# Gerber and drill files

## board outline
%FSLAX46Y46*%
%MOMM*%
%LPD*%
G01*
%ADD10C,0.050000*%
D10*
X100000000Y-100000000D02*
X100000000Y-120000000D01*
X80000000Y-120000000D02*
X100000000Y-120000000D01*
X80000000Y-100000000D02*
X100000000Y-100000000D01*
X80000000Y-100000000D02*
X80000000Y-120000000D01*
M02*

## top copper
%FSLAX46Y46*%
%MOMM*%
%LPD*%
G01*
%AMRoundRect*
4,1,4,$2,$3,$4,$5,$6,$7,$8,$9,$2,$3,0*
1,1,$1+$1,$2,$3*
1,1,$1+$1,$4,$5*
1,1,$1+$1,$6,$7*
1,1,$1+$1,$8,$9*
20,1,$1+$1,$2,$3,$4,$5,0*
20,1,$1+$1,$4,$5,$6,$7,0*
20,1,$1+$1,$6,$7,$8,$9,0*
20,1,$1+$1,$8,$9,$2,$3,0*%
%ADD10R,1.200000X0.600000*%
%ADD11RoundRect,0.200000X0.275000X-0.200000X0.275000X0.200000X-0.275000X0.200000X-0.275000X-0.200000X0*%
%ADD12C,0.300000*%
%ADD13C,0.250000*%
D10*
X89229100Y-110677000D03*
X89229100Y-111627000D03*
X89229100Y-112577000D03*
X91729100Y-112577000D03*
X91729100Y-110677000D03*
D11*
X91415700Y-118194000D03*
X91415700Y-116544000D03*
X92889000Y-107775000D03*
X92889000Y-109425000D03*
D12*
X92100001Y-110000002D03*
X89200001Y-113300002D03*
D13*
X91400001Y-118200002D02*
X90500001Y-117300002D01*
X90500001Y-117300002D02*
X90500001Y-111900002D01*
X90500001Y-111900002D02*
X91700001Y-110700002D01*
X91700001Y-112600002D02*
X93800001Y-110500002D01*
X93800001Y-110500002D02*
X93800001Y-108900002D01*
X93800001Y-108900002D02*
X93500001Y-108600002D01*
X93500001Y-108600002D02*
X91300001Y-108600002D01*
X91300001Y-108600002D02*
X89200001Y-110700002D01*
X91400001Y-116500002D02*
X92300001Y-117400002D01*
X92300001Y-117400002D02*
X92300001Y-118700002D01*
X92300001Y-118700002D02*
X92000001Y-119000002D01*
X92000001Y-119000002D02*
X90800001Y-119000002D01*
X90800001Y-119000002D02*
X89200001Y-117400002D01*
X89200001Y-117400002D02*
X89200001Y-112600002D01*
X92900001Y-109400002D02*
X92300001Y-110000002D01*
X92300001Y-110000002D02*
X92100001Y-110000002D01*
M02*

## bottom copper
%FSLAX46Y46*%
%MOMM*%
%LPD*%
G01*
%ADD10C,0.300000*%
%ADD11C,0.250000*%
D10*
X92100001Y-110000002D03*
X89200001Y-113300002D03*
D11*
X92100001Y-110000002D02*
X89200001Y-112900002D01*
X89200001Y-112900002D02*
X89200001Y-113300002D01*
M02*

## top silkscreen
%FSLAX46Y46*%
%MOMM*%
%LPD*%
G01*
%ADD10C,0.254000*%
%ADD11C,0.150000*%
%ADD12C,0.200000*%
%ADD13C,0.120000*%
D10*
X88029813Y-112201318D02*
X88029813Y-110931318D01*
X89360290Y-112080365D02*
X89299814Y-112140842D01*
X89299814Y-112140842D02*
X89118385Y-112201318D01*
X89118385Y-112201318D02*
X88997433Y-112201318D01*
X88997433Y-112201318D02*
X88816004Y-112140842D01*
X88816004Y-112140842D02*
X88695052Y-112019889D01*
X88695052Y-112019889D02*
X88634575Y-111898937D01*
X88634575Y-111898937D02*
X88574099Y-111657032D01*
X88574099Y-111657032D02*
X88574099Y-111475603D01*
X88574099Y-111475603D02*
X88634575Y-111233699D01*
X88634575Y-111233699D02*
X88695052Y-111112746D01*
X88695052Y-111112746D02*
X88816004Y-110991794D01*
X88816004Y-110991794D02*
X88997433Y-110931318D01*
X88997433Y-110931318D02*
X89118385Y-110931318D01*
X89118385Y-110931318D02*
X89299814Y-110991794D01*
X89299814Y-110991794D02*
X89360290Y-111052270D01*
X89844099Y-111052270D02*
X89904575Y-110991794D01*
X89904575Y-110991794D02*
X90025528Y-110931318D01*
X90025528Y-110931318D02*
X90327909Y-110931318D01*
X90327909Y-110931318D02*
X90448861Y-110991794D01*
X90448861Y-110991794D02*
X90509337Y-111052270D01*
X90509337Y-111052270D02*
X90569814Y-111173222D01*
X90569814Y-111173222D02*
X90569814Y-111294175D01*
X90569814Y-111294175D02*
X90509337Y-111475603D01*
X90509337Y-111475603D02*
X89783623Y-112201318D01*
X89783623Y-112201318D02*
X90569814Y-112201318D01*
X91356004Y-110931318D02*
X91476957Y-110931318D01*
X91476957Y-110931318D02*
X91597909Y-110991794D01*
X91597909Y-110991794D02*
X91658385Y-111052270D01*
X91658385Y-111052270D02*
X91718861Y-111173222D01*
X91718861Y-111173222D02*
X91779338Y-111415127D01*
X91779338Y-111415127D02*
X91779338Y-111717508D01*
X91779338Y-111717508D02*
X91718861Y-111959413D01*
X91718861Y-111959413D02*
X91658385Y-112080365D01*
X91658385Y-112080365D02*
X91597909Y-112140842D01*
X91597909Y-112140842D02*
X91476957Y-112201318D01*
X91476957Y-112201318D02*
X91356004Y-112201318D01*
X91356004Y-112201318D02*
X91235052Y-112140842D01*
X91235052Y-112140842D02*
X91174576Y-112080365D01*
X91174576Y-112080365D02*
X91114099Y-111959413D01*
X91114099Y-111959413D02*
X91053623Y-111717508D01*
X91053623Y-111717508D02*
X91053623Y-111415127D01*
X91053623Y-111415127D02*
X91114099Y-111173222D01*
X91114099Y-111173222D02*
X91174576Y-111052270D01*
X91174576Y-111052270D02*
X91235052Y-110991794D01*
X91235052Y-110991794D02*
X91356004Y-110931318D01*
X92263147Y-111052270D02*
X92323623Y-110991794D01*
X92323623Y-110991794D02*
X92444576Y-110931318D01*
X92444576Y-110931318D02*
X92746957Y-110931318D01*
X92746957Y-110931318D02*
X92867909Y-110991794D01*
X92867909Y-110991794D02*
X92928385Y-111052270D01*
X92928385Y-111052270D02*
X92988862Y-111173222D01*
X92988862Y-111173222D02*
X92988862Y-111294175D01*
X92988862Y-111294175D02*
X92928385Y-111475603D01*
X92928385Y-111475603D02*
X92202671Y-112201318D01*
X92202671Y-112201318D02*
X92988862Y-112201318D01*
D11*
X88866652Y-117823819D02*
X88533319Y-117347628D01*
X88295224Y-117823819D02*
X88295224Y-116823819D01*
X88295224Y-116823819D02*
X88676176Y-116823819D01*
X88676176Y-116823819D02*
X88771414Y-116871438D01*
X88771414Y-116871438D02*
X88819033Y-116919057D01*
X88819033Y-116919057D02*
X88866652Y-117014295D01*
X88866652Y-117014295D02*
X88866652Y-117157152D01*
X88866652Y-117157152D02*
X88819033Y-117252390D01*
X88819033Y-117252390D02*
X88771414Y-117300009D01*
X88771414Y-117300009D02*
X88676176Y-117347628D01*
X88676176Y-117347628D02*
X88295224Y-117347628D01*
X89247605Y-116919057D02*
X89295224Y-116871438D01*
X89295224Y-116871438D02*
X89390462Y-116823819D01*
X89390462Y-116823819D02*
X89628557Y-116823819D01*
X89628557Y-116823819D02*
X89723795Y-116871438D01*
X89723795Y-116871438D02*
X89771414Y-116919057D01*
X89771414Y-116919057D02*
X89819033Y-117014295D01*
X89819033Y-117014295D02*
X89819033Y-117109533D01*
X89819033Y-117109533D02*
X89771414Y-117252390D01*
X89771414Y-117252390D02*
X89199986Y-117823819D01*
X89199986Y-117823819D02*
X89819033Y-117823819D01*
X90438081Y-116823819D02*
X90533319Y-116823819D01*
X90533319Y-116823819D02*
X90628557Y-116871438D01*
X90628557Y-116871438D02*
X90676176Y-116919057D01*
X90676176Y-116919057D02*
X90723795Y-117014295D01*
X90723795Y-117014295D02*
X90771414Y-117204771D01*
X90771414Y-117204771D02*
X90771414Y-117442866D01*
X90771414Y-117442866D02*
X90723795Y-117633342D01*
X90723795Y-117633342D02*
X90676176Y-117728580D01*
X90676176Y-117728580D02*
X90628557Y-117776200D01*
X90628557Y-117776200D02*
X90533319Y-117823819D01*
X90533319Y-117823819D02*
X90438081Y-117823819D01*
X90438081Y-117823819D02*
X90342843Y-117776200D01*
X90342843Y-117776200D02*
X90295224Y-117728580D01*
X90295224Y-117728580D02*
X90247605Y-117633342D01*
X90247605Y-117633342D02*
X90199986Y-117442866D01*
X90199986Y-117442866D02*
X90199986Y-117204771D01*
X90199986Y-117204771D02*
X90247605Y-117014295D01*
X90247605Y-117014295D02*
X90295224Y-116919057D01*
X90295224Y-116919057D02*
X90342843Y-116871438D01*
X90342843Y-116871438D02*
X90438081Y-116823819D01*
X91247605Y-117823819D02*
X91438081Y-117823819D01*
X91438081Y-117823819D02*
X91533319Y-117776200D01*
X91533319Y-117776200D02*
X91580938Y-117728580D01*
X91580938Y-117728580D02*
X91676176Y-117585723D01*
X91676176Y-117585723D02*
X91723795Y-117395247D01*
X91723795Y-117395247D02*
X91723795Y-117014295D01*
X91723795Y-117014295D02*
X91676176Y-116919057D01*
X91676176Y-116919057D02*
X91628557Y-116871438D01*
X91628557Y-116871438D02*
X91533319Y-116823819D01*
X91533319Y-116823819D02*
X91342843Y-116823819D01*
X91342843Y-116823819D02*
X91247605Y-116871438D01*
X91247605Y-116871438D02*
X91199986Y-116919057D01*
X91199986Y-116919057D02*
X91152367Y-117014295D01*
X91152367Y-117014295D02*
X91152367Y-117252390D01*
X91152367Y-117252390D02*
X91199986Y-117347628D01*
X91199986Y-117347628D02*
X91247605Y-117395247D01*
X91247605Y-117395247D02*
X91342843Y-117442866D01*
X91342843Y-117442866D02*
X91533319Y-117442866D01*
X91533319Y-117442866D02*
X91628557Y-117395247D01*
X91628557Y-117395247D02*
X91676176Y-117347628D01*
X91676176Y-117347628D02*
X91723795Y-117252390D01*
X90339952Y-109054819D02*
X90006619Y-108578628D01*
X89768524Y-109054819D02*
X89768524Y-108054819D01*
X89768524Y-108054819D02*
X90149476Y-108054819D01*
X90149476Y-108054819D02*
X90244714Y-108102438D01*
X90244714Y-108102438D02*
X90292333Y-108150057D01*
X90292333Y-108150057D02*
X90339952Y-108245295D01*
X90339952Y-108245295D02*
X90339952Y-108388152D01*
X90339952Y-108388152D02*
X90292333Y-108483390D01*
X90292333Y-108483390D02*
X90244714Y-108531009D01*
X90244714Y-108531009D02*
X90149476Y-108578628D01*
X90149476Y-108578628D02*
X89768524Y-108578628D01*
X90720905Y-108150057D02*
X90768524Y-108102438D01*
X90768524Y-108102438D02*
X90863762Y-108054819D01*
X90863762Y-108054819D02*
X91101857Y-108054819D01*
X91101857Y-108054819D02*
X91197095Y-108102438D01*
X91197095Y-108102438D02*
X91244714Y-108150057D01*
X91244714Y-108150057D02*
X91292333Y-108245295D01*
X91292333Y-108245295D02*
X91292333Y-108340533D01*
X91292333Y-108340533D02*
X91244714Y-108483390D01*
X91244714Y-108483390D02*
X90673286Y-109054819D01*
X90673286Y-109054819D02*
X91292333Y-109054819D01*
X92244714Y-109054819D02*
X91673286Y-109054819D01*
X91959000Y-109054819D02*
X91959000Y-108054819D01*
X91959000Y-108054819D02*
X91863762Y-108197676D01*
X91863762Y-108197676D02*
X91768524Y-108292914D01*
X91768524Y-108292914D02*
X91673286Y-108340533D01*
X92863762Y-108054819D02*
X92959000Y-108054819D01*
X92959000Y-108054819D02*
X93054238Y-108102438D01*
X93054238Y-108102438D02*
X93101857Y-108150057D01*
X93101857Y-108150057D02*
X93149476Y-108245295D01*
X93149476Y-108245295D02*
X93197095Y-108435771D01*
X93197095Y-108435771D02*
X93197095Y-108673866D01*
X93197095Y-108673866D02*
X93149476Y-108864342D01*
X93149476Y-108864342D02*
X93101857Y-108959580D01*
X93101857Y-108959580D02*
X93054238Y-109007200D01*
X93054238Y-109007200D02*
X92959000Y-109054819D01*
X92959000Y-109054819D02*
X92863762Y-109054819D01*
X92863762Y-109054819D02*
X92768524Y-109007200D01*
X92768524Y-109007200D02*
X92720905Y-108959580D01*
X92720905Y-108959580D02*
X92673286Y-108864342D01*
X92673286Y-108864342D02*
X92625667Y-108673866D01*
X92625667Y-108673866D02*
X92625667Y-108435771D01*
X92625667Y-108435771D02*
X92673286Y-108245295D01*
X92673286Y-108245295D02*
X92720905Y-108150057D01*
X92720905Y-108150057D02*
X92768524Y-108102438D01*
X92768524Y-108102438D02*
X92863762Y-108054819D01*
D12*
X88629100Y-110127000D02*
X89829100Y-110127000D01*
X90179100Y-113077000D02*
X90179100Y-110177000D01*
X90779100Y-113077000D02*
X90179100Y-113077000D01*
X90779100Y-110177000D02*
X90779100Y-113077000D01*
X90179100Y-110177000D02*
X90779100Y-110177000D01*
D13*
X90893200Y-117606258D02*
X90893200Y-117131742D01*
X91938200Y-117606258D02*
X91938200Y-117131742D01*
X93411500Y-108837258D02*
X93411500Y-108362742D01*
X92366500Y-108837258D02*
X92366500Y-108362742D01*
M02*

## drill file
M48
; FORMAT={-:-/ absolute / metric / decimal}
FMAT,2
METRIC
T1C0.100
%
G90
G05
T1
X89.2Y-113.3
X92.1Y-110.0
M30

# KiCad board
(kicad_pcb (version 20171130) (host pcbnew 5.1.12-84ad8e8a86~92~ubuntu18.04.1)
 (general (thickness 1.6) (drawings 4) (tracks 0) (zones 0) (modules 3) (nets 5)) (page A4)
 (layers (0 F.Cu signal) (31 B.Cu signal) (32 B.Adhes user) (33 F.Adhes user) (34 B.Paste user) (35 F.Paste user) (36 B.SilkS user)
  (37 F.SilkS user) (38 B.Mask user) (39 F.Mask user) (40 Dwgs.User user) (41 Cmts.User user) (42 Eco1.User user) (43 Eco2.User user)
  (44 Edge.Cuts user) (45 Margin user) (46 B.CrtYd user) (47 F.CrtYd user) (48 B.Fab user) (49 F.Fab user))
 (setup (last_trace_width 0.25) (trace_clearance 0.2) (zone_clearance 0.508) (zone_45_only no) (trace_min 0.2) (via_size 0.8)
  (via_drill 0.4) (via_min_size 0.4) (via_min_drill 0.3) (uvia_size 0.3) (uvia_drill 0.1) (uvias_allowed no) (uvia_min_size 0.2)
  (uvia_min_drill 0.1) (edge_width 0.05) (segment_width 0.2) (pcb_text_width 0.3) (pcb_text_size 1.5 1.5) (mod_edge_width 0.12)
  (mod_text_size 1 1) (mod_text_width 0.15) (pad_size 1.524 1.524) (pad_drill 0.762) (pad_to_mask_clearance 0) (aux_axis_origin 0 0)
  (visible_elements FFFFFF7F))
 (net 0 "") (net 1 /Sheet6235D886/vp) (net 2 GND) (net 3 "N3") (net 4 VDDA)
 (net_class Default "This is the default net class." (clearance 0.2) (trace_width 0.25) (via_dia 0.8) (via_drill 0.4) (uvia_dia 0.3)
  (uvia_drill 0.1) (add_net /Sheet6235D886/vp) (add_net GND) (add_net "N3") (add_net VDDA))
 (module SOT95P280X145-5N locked (layer F.Cu) (at 90.479100 111.627000)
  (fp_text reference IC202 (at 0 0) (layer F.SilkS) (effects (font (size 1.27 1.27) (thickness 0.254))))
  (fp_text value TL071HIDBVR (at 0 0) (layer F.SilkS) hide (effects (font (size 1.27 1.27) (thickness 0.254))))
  (fp_line (start -1.85 -1.5) (end -0.65 -1.5) (layer F.SilkS) (width 0.2))
  (fp_line (start -0.3 1.45) (end -0.3 -1.45) (layer F.SilkS) (width 0.2))
  (fp_line (start 0.3 1.45) (end -0.3 1.45) (layer F.SilkS) (width 0.2))
  (fp_line (start 0.3 -1.45) (end 0.3 1.45) (layer F.SilkS) (width 0.2))
  (fp_line (start -0.3 -1.45) (end 0.3 -1.45) (layer F.SilkS) (width 0.2))
  (pad 1 smd rect (at -1.25 -0.95 90.000000) (size 0.6 1.2) (layers F.Cu F.Mask F.Paste) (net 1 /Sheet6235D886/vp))
  (pad 2 smd rect (at -1.25 0 90.000000) (size 0.6 1.2) (layers F.Cu F.Mask F.Paste) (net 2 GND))
  (pad 3 smd rect (at -1.25 0.95 90.000000) (size 0.6 1.2) (layers F.Cu F.Mask F.Paste) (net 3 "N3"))
  (pad 4 smd rect (at 1.25 0.95 90.000000) (size 0.6 1.2) (layers F.Cu F.Mask F.Paste) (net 1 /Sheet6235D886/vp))
  (pad 5 smd rect (at 1.25 -0.95 90.000000) (size 0.6 1.2) (layers F.Cu F.Mask F.Paste) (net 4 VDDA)))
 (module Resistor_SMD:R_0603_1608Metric (layer F.Cu) (at 91.415700 117.369000 90.000000)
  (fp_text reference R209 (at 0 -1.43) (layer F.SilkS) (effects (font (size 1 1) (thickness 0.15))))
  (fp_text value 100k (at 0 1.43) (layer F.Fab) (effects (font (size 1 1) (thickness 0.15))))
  (fp_line (start -0.237258 -0.5225) (end 0.237258 -0.5225) (layer F.SilkS) (width 0.12))
  (fp_line (start -0.237258 0.5225) (end 0.237258 0.5225) (layer F.SilkS) (width 0.12))
  (pad 1 smd roundrect (at -0.825 0 90.000000) (size 0.8 0.95) (layers F.Cu F.Mask F.Paste) (roundrect_rratio 0.25) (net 4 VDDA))
  (pad 2 smd roundrect (at 0.825 0 90.000000) (size 0.8 0.95) (layers F.Cu F.Mask F.Paste) (roundrect_rratio 0.25) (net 3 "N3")))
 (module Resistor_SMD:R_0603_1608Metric (layer F.Cu) (at 92.889000 108.600000 90.000000)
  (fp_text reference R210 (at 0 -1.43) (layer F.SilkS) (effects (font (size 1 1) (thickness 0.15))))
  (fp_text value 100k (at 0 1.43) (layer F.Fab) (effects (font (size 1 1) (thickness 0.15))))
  (fp_line (start -0.237258 0.5225) (end 0.237258 0.5225) (layer F.SilkS) (width 0.12))
  (fp_line (start -0.237258 -0.5225) (end 0.237258 -0.5225) (layer F.SilkS) (width 0.12))
  (pad 2 smd roundrect (at 0.825 0 90.000000) (size 0.8 0.95) (layers F.Cu F.Mask F.Paste) (roundrect_rratio 0.25) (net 2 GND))
  (pad 1 smd roundrect (at -0.825 0 90.000000) (size 0.8 0.95) (layers F.Cu F.Mask F.Paste) (roundrect_rratio 0.25) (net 3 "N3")))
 (gr_line (start 100 100) (end 100 120) (layer Edge.Cuts) (width 0.05))
 (gr_line (start 80 120) (end 100 120) (layer Edge.Cuts) (width 0.05))
 (gr_line (start 80 100) (end 100 100) (layer Edge.Cuts) (width 0.05))
 (gr_line (start 80 100) (end 80 120) (layer Edge.Cuts) (width 0.05))
 (segment (start 91.400001 118.200002) (end 90.500001 117.300002) (width 0.250000) (layer F.Cu) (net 4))
 (segment (start 90.500001 117.300002) (end 90.500001 111.900002) (width 0.250000) (layer F.Cu) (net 4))
 (segment (start 90.500001 111.900002) (end 91.700001 110.700002) (width 0.250000) (layer F.Cu) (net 4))
 (segment (start 91.700001 112.600002) (end 93.800001 110.500002) (width 0.250000) (layer F.Cu) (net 1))
 (segment (start 93.800001 110.500002) (end 93.800001 108.900002) (width 0.250000) (layer F.Cu) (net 1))
 (segment (start 93.800001 108.900002) (end 93.500001 108.600002) (width 0.250000) (layer F.Cu) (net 1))
 (segment (start 93.500001 108.600002) (end 91.300001 108.600002) (width 0.250000) (layer F.Cu) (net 1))
 (segment (start 91.300001 108.600002) (end 89.200001 110.700002) (width 0.250000) (layer F.Cu) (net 1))
 (segment (start 91.400001 116.500002) (end 92.300001 117.400002) (width 0.250000) (layer F.Cu) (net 3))
 (segment (start 92.300001 117.400002) (end 92.300001 118.700002) (width 0.250000) (layer F.Cu) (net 3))
 (segment (start 92.300001 118.700002) (end 92.000001 119.000002) (width 0.250000) (layer F.Cu) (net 3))
 (segment (start 92.000001 119.000002) (end 90.800001 119.000002) (width 0.250000) (layer F.Cu) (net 3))
 (segment (start 90.800001 119.000002) (end 89.200001 117.400002) (width 0.250000) (layer F.Cu) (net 3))
 (segment (start 89.200001 117.400002) (end 89.200001 112.600002) (width 0.250000) (layer F.Cu) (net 3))
 (segment (start 92.900001 109.400002) (end 92.300001 110.000002) (width 0.250000) (layer F.Cu) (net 3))
 (segment (start 92.300001 110.000002) (end 92.100001 110.000002) (width 0.250000) (layer F.Cu) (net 3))
 (segment (start 92.100001 110.000002) (end 89.200001 112.900002) (width 0.250000) (layer B.Cu) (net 3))
 (segment (start 89.200001 112.900002) (end 89.200001 113.300002) (width 0.250000) (layer B.Cu) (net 3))
 (via micro (at 92.100001 110.000002) (size 0.300000) (drill 0.100000) (layers F.Cu B.Cu) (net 3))
 (via micro (at 89.200001 113.300002) (size 0.300000) (drill 0.100000) (layers F.Cu B.Cu) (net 3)))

